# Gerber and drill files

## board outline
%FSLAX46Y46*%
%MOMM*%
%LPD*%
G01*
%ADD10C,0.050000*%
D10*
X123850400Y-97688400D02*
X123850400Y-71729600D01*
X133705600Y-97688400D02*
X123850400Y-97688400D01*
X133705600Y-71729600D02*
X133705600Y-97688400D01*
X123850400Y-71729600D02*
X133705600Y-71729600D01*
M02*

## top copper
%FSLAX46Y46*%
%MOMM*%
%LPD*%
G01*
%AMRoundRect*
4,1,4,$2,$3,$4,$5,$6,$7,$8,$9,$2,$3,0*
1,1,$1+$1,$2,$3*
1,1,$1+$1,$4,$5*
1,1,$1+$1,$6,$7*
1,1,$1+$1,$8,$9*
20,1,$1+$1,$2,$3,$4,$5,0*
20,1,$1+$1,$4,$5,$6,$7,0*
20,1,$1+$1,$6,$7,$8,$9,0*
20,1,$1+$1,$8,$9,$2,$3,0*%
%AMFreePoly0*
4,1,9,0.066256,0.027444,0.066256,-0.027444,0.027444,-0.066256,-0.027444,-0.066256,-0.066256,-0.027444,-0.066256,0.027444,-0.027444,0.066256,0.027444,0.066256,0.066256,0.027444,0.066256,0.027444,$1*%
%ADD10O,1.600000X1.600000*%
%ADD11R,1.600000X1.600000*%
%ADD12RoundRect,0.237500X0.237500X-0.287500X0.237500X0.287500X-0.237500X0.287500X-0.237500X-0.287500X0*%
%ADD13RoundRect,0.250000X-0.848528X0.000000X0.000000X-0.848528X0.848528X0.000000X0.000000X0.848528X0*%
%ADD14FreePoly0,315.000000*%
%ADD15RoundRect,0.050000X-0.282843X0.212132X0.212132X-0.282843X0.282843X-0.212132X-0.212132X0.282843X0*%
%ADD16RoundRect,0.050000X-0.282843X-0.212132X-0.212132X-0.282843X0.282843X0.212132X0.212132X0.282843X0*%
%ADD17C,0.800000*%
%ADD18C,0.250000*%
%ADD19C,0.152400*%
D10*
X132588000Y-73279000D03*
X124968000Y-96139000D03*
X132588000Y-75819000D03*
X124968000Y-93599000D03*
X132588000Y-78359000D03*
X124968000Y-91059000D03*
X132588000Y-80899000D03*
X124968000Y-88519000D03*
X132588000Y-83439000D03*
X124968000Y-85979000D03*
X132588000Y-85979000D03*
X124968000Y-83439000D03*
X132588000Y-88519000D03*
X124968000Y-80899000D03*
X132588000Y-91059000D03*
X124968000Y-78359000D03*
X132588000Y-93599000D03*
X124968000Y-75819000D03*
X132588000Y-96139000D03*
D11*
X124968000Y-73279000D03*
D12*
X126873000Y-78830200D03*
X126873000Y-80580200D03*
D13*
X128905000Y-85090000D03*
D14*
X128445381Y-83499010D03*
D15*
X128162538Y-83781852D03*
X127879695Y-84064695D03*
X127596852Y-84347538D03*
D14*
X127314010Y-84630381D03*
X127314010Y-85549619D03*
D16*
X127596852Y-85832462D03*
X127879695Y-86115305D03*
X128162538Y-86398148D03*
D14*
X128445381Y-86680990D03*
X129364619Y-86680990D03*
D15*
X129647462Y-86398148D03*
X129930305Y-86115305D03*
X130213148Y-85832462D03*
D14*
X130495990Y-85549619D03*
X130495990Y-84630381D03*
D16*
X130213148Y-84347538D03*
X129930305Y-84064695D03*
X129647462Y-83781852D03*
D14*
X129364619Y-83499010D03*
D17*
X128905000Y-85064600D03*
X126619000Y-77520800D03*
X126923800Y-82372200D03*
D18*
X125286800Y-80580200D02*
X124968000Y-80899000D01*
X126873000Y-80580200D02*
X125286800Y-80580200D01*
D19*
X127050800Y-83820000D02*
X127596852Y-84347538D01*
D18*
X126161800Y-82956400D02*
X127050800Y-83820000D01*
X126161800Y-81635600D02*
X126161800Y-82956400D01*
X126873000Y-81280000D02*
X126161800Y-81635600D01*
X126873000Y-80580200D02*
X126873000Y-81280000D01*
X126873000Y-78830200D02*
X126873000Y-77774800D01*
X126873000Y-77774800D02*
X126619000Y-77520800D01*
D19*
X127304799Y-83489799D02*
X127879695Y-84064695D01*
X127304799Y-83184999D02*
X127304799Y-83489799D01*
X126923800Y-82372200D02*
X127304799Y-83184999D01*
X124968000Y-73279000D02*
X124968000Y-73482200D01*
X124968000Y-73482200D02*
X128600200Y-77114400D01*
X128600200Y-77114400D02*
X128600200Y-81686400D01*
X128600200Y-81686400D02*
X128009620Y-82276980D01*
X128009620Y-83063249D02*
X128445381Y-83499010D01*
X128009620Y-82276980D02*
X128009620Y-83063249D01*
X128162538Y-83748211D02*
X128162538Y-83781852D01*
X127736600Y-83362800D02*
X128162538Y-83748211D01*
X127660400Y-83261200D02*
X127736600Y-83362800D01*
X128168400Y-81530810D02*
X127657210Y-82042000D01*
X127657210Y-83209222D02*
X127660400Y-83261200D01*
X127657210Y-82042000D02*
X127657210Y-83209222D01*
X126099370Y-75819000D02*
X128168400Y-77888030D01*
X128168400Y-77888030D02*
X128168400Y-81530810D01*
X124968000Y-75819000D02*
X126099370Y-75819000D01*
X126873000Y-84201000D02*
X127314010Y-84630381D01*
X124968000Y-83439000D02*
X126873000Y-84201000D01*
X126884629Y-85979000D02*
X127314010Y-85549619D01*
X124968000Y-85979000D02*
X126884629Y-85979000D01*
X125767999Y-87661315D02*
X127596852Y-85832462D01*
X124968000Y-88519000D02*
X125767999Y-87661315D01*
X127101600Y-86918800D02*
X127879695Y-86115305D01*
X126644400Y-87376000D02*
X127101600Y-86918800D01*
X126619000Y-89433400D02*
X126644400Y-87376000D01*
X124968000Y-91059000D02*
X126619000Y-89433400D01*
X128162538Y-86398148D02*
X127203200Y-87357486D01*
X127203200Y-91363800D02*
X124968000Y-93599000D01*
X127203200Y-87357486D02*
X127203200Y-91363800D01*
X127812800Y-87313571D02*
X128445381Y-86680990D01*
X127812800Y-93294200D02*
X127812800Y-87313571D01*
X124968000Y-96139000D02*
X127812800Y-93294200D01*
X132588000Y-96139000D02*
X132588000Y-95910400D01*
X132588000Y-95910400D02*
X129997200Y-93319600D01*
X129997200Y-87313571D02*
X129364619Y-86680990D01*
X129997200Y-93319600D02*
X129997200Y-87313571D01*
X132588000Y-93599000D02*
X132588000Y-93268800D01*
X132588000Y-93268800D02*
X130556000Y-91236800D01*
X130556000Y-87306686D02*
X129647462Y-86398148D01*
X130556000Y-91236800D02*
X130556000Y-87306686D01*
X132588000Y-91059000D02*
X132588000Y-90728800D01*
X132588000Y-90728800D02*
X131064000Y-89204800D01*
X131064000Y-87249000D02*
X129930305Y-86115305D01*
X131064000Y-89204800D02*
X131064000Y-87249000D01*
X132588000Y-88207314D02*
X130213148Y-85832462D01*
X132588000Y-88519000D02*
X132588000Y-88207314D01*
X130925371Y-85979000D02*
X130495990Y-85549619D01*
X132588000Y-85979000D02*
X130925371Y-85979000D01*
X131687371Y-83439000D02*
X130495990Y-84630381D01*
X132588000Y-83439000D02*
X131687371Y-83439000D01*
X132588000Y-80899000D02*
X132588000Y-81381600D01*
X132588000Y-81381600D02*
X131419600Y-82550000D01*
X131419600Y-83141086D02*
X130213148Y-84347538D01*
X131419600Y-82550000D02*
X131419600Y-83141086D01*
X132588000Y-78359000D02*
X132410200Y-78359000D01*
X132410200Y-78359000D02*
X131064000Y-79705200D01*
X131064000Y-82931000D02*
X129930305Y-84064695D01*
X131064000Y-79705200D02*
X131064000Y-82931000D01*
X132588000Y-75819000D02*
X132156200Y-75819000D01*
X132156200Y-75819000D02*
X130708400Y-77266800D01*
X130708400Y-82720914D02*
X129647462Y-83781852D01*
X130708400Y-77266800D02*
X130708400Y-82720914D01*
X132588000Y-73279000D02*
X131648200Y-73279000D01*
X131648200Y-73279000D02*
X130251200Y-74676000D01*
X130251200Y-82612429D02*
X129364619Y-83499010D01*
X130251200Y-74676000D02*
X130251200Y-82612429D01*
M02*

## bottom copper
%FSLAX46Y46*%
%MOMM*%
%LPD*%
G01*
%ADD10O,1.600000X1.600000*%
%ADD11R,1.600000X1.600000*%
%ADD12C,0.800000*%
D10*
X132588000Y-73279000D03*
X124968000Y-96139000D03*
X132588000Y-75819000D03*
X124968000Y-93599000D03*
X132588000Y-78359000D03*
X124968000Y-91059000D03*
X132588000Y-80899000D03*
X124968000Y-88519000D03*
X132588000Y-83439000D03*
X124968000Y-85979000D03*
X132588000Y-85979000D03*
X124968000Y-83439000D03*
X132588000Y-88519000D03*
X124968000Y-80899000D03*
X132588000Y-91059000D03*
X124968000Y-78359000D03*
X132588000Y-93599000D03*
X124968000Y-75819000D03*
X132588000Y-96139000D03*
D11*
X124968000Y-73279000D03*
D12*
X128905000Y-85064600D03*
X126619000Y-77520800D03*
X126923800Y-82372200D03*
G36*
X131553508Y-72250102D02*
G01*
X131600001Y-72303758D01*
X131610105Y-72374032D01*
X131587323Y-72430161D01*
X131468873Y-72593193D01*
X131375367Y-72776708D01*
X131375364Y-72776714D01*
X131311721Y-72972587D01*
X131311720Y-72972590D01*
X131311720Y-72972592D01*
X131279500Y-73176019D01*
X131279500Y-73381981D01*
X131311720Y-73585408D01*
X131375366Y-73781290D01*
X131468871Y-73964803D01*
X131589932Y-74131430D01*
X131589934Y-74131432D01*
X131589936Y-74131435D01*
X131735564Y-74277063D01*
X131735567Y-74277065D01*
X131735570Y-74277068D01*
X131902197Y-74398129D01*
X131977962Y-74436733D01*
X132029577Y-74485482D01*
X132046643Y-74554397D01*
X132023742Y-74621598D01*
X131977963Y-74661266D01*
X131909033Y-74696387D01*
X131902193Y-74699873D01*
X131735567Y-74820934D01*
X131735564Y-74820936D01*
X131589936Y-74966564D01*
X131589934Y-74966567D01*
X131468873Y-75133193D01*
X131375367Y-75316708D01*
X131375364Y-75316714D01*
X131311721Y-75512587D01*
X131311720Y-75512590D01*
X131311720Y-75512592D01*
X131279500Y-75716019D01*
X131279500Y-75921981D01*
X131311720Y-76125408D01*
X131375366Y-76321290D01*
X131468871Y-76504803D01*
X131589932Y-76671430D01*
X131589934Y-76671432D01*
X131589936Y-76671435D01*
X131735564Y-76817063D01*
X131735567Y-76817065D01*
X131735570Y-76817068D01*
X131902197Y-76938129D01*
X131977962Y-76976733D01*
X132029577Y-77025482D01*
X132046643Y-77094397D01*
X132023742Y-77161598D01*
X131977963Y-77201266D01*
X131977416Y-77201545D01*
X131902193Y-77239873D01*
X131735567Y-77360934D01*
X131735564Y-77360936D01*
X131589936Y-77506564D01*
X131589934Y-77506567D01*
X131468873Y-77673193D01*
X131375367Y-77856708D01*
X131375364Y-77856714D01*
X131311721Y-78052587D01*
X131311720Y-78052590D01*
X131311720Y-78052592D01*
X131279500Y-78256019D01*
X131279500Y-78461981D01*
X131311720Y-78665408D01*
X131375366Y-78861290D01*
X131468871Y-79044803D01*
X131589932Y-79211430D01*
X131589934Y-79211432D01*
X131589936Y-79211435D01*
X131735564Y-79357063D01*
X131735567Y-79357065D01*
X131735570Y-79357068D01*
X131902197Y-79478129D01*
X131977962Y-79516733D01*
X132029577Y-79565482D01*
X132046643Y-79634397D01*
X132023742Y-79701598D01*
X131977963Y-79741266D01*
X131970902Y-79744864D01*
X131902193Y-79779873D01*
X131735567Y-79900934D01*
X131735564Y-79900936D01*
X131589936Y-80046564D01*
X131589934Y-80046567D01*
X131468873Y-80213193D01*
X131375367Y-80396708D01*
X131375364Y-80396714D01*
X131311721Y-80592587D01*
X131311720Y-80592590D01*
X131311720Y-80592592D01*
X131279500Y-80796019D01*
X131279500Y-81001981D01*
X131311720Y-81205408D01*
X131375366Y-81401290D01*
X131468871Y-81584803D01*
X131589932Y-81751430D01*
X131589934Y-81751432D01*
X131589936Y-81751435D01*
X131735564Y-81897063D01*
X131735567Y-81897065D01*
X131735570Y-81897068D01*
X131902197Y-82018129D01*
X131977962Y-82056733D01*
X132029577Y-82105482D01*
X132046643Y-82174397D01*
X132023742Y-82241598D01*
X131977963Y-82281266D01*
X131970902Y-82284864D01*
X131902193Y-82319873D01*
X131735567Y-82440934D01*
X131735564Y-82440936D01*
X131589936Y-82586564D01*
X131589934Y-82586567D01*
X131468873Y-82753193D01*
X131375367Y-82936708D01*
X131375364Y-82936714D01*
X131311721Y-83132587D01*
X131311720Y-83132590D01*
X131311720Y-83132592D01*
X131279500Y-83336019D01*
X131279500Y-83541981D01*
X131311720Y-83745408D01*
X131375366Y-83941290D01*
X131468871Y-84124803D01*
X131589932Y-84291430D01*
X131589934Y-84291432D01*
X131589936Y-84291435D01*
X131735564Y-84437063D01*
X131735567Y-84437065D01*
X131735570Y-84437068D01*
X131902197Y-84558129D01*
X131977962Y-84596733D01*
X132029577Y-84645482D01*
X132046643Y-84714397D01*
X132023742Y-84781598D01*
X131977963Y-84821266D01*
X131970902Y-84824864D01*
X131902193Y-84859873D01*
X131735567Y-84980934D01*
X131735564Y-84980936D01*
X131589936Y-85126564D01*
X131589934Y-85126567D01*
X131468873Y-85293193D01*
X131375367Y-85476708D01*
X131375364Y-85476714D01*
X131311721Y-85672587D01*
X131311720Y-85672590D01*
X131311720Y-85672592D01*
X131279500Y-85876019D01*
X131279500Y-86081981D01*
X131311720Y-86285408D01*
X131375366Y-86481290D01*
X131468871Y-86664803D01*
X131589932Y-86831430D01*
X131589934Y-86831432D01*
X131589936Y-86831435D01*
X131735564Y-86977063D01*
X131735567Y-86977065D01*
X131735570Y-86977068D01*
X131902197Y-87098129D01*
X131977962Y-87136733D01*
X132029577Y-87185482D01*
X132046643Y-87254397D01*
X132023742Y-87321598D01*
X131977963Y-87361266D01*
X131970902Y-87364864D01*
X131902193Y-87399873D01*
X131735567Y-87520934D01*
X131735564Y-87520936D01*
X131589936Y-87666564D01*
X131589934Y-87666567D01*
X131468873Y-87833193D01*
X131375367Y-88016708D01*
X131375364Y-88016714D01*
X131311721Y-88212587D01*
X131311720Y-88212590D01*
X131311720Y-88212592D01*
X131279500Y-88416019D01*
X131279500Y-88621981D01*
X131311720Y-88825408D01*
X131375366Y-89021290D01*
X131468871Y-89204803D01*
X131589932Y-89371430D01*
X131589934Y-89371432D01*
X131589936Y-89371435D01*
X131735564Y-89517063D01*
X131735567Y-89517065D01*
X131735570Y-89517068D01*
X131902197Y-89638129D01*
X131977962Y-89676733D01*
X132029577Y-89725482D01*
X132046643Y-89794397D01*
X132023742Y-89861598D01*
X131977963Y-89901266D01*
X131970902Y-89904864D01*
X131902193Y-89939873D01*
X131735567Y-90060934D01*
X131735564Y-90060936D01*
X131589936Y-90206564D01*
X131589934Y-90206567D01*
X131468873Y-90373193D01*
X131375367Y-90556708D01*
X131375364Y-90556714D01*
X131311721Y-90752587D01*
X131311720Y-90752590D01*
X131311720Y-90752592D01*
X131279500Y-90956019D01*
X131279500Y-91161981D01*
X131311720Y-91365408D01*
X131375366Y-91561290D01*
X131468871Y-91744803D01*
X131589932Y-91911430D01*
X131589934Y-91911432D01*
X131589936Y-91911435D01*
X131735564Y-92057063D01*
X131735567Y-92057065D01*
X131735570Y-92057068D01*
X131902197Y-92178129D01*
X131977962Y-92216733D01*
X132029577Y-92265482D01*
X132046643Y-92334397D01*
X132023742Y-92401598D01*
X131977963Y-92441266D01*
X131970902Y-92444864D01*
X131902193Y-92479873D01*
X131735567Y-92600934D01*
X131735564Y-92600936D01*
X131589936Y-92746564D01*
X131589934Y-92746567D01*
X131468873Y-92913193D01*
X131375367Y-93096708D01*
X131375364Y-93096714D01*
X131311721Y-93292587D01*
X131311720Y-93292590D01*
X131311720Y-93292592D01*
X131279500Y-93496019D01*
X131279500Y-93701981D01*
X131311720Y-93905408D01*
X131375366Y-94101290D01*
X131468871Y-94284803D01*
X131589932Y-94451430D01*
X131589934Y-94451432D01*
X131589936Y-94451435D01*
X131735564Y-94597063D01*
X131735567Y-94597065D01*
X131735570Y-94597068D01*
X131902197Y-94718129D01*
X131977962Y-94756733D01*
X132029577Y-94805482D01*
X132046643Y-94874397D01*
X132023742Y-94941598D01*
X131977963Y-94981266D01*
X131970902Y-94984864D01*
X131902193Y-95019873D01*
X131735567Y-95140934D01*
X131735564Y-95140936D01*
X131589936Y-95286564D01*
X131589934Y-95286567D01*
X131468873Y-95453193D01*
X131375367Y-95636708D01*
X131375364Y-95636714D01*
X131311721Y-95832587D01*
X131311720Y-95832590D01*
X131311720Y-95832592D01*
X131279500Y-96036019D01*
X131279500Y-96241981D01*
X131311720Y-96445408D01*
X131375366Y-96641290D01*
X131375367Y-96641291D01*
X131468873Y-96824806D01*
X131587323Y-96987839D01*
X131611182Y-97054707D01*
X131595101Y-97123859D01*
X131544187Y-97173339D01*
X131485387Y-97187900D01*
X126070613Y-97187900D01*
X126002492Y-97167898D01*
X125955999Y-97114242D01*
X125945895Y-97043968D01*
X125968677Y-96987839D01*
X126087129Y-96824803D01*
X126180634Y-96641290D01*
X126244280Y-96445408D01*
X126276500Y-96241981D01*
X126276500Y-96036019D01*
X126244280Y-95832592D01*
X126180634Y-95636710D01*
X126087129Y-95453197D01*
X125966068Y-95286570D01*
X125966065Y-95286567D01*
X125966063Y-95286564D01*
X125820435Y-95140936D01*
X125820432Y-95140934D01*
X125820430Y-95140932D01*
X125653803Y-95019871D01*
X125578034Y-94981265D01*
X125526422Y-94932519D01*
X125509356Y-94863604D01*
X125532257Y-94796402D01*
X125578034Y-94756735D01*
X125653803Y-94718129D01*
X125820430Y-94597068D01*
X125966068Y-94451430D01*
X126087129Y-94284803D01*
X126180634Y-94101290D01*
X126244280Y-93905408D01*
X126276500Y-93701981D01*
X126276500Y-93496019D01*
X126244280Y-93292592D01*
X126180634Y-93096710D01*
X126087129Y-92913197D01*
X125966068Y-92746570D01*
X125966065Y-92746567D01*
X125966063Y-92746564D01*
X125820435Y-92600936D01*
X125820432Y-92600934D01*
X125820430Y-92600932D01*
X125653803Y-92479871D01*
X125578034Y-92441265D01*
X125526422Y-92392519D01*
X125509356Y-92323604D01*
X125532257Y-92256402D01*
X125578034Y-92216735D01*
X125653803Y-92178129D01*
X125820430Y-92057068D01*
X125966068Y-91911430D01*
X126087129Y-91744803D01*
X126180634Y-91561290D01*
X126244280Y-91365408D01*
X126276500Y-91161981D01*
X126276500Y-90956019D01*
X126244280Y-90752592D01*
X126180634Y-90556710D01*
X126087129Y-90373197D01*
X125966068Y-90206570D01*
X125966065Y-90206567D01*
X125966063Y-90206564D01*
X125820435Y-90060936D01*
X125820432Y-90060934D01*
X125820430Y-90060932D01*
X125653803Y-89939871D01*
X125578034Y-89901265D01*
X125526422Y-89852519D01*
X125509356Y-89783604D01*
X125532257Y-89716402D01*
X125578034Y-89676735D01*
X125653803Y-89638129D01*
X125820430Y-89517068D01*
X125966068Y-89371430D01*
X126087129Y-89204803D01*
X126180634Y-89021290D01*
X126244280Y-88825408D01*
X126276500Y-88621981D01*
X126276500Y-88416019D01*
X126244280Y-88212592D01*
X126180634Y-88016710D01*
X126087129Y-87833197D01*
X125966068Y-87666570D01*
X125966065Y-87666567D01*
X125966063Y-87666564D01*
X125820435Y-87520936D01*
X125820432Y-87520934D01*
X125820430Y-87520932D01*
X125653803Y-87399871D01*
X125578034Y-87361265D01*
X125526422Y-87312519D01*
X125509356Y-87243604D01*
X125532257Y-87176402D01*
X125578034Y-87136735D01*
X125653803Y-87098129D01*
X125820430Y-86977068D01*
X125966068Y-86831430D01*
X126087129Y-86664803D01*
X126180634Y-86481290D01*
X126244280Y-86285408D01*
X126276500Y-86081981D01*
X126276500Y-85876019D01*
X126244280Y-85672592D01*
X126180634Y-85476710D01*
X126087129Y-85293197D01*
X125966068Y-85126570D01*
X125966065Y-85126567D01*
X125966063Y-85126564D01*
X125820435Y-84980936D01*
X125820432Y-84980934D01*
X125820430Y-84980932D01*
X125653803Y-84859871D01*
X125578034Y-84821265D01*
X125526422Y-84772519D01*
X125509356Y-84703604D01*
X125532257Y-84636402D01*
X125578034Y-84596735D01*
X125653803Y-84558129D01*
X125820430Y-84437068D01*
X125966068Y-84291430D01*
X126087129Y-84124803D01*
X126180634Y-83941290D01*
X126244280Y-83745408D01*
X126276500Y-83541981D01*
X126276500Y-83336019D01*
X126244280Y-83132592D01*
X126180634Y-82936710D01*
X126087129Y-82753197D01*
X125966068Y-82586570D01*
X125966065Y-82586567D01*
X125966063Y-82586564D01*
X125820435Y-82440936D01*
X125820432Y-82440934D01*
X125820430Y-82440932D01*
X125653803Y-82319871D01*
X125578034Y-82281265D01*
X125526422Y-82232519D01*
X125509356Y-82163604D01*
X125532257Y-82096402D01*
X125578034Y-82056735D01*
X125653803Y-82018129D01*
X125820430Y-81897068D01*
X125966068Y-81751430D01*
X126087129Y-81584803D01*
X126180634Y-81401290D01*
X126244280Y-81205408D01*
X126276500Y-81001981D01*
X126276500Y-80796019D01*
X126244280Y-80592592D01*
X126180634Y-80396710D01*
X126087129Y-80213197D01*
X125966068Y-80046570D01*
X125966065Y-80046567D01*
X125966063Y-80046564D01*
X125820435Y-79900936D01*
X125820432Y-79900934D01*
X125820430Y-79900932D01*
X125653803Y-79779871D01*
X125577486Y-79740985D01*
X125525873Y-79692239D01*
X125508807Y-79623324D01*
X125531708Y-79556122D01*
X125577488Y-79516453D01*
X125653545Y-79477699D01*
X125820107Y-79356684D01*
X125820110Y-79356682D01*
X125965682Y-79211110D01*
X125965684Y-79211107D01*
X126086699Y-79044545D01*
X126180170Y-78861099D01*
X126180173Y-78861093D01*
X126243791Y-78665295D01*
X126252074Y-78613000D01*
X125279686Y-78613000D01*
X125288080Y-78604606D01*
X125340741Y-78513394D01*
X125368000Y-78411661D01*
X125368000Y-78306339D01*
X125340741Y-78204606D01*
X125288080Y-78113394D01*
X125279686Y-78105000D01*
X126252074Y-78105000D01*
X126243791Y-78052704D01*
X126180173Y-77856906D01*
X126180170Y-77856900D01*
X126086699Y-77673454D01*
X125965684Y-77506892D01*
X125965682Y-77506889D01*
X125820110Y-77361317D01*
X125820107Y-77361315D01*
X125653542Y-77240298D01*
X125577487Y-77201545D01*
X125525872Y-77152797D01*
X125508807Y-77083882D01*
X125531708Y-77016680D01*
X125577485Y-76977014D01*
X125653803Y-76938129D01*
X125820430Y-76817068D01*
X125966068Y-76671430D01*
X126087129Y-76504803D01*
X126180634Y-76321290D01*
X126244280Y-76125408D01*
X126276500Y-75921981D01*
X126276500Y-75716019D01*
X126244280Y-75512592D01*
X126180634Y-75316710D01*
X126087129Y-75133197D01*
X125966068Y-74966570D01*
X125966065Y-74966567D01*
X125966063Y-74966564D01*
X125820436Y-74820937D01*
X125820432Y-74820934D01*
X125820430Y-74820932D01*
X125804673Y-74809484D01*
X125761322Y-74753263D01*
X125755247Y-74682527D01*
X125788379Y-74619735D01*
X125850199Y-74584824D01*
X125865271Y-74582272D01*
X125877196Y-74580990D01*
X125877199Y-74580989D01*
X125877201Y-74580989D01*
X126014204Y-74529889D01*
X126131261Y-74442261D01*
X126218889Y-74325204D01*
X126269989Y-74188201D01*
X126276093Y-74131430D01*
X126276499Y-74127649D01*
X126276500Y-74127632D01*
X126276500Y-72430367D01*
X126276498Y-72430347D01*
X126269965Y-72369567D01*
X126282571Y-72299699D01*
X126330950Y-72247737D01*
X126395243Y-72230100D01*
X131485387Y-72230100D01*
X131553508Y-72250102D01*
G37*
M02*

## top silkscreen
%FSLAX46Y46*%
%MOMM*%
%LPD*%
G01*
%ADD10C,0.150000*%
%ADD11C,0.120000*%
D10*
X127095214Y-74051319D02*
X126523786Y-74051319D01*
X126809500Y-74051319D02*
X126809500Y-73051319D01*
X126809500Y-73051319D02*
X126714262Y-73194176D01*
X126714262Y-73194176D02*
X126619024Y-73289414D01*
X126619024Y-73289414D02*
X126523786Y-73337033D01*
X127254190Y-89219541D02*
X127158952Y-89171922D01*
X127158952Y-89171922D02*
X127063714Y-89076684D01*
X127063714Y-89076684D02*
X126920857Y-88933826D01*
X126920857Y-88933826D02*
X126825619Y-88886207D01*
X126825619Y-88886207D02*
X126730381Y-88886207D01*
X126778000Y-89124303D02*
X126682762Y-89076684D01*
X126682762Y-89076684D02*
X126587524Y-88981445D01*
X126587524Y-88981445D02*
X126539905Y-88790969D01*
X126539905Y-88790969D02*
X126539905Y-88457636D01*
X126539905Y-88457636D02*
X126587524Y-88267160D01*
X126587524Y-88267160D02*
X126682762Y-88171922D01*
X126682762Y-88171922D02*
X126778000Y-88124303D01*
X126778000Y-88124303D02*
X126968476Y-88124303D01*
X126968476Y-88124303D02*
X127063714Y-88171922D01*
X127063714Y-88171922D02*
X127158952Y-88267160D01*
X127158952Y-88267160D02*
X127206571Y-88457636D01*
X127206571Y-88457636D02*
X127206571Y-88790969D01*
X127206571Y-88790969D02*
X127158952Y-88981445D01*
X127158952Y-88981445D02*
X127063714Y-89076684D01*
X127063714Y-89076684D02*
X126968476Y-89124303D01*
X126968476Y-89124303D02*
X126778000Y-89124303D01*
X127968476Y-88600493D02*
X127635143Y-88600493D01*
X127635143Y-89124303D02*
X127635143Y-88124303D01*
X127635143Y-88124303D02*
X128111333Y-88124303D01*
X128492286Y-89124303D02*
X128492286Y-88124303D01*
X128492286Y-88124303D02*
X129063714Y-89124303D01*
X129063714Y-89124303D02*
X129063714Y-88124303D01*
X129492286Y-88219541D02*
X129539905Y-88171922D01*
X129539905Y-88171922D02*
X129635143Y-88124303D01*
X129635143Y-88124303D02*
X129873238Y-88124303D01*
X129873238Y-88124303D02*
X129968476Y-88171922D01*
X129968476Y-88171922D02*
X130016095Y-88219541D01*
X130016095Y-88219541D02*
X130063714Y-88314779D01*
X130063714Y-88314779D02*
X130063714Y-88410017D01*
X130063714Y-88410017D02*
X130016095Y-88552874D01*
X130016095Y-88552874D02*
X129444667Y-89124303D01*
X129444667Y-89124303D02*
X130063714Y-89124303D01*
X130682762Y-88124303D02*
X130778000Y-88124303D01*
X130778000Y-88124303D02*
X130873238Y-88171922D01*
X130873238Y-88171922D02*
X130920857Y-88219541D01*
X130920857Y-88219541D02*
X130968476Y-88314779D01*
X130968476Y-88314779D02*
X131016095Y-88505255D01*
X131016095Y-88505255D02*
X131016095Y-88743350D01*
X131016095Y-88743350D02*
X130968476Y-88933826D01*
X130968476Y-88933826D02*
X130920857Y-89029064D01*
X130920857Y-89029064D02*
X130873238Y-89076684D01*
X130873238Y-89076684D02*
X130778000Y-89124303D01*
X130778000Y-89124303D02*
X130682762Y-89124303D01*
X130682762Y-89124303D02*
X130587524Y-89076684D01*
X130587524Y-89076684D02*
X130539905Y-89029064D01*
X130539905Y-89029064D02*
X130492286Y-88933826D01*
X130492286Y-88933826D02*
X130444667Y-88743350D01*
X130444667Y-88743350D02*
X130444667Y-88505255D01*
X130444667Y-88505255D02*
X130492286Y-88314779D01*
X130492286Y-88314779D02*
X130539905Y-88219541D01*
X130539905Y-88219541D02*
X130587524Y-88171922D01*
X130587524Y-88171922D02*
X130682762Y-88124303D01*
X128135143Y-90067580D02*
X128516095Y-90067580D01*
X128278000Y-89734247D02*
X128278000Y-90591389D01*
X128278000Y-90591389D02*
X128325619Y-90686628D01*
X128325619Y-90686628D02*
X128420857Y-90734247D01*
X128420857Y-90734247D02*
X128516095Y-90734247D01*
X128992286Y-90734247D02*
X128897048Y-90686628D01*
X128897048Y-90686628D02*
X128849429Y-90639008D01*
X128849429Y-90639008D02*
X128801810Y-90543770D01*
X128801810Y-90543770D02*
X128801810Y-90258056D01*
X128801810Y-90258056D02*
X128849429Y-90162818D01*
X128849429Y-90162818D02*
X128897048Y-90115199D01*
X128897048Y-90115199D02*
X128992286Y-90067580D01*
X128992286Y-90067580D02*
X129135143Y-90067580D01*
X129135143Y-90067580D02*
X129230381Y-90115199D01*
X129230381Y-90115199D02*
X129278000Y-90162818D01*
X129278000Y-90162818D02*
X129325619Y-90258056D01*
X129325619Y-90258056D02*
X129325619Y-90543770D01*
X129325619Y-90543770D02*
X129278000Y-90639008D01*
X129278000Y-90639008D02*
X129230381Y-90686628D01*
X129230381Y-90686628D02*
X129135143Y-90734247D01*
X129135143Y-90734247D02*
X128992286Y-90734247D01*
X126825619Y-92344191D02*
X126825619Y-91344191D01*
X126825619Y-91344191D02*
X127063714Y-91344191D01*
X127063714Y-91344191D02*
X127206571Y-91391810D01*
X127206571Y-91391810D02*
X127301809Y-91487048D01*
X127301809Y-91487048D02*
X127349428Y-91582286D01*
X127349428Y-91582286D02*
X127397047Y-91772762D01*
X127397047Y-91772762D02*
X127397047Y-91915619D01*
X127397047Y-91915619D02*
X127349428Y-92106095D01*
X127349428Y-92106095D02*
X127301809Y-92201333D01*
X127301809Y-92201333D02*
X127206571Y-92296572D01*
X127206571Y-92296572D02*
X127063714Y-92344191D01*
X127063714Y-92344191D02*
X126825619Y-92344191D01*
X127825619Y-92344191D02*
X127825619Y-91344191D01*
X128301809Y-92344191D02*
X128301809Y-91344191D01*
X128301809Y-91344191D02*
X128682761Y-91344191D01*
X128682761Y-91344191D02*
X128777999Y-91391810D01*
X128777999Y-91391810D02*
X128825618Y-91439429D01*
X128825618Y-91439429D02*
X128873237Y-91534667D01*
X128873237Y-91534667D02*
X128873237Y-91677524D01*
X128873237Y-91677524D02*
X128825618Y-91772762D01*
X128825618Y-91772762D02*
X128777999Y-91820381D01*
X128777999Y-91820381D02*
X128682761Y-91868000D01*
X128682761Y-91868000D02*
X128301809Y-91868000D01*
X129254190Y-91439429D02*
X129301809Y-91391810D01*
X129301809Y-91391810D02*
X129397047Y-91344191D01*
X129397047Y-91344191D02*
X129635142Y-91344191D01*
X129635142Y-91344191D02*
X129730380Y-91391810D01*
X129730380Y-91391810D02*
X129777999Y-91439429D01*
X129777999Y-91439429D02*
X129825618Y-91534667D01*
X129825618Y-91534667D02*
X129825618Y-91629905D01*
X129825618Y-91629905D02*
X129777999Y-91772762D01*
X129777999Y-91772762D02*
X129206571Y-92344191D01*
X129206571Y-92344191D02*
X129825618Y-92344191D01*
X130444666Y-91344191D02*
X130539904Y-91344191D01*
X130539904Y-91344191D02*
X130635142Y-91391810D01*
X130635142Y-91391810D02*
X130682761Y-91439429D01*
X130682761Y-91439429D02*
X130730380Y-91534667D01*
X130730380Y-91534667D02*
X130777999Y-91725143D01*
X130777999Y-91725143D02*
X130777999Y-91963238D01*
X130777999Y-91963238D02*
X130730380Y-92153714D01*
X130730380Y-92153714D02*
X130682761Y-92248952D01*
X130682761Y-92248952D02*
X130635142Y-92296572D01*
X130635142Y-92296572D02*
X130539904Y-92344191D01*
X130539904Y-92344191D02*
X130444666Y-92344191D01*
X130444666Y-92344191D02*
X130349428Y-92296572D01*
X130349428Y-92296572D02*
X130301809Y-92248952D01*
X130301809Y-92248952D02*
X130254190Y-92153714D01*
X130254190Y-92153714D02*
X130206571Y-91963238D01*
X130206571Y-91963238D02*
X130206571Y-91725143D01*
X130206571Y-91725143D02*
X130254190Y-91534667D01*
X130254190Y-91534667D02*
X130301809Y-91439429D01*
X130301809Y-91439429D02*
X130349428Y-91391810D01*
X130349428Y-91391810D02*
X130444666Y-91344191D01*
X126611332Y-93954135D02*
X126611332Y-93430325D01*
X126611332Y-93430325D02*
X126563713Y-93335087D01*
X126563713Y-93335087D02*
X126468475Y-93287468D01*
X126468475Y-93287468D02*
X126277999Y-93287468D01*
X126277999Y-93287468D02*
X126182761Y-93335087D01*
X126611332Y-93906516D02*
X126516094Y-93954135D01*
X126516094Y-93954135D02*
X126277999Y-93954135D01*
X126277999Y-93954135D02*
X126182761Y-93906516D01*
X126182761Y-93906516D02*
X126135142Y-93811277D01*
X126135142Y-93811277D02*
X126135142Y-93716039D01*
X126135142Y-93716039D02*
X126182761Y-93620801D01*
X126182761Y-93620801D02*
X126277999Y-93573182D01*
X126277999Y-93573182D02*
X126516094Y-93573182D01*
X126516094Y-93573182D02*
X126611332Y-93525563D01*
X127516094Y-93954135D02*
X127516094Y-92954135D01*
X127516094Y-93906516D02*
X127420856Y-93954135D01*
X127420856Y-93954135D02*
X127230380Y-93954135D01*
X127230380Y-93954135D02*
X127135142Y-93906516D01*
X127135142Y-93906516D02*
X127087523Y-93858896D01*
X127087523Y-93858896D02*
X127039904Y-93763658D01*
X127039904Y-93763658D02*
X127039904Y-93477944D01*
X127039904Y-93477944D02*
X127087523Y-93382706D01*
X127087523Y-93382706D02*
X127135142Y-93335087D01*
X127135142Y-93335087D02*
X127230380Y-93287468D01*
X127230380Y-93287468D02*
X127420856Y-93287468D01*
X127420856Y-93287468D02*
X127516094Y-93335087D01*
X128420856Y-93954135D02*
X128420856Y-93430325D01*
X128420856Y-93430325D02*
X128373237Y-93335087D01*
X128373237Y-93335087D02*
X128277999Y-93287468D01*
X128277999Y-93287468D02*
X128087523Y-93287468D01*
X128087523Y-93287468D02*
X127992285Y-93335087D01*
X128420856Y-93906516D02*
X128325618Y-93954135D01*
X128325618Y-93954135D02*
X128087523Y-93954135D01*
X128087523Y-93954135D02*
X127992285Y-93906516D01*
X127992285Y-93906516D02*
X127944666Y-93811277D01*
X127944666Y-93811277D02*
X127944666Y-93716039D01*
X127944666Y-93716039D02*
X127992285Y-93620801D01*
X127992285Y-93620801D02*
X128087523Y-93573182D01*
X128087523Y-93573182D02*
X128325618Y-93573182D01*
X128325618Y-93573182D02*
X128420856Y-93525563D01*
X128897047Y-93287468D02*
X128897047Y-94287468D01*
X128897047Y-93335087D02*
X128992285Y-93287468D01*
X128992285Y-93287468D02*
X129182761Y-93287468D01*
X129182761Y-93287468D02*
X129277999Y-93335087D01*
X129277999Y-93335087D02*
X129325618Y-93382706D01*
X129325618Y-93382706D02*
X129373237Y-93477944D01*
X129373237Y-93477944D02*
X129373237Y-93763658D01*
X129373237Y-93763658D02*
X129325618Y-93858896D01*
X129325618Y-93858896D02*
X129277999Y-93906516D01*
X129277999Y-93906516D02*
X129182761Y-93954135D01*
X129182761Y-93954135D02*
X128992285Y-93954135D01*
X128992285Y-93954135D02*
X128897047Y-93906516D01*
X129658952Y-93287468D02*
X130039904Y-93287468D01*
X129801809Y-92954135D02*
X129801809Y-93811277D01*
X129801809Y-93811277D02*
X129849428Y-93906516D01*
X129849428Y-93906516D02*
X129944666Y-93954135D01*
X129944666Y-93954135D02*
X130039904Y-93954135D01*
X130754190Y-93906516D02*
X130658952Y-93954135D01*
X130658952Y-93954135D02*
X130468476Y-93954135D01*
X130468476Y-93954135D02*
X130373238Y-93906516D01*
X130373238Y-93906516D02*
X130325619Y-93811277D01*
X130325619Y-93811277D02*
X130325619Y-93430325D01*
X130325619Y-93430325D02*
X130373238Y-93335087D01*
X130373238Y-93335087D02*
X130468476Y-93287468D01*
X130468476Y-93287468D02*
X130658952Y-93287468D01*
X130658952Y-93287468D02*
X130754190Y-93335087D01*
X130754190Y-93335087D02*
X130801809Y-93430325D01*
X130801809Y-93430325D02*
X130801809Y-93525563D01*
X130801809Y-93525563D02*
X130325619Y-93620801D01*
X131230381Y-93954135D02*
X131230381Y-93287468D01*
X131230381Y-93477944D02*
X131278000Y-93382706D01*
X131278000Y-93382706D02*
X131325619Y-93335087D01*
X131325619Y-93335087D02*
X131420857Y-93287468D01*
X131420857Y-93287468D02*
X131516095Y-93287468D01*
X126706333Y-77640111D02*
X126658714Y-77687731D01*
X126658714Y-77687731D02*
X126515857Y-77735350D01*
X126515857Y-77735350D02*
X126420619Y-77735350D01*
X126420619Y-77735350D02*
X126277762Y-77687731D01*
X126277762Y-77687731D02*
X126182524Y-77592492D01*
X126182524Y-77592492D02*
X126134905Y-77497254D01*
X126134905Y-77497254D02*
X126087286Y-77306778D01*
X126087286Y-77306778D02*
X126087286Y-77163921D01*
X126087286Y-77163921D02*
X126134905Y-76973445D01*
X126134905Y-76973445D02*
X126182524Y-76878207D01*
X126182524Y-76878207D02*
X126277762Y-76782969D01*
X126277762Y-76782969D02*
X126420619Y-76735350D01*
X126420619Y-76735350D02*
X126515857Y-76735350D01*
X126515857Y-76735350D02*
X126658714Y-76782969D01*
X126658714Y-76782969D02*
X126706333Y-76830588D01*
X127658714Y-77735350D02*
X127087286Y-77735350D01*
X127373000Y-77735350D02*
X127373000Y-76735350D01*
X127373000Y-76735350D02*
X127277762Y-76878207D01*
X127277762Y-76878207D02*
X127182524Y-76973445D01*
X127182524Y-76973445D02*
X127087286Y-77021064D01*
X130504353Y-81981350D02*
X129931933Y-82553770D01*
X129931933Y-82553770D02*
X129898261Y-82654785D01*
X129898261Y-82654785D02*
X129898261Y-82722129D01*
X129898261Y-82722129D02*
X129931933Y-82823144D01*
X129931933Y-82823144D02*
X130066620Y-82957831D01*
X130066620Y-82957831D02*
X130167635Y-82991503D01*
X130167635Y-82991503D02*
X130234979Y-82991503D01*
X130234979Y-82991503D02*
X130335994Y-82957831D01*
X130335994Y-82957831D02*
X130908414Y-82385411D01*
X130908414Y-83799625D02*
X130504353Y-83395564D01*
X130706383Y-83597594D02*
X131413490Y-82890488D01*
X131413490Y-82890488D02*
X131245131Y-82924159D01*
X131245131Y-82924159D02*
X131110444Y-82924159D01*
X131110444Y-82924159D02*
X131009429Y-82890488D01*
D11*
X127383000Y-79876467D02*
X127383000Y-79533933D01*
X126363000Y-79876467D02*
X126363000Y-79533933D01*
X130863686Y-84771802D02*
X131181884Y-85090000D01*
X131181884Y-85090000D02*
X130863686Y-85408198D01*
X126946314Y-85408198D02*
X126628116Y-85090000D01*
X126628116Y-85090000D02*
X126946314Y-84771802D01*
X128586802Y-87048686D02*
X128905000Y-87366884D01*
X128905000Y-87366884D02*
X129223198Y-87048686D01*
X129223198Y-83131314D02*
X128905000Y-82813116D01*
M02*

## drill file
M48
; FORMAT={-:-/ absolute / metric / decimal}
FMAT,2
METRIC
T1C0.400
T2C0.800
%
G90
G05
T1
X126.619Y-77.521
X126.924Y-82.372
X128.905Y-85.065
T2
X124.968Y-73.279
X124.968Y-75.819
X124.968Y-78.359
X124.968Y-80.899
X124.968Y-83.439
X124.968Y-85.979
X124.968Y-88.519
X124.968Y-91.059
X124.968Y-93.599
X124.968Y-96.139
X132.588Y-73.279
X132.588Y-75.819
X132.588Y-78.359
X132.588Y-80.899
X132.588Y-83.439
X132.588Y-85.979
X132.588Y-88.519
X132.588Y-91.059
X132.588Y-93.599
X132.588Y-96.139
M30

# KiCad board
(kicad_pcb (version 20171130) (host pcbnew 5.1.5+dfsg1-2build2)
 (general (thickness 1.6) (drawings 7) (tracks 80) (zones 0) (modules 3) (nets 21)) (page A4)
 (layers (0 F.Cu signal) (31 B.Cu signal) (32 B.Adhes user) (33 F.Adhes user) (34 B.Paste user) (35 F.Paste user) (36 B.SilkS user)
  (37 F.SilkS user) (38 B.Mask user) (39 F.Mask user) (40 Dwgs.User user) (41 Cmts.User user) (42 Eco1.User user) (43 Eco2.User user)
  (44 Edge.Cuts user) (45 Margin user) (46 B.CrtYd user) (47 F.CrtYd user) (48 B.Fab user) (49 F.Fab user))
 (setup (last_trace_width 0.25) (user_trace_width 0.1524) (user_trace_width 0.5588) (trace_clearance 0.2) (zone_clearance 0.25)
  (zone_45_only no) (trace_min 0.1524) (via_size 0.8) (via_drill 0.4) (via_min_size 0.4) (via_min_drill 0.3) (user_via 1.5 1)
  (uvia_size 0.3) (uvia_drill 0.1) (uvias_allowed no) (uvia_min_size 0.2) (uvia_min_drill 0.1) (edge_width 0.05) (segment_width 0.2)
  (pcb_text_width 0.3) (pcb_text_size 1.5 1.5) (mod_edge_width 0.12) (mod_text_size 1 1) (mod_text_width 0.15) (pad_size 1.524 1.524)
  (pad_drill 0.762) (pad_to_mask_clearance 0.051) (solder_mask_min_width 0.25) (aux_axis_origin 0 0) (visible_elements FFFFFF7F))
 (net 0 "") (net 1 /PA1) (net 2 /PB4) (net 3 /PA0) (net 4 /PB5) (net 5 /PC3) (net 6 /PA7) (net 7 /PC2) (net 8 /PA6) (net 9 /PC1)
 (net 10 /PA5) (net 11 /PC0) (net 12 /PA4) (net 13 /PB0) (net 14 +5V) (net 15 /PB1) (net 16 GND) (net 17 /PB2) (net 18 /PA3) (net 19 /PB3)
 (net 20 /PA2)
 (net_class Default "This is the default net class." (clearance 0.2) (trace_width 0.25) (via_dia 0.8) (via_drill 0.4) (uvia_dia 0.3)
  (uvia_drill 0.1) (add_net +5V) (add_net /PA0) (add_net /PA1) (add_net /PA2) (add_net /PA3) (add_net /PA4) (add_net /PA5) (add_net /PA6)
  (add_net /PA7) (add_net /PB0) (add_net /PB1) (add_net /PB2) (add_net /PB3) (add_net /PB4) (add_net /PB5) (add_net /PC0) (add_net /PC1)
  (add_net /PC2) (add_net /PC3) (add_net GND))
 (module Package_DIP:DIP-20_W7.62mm (layer F.Cu) (at 124.968 73.279)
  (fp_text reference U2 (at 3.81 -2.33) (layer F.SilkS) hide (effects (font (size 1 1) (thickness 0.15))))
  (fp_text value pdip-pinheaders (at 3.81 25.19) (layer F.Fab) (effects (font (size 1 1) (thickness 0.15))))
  (pad 20 thru_hole oval (at 7.62 0) (size 1.6 1.6) (drill 0.8) (layers *.Cu *.Mask) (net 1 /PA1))
  (pad 10 thru_hole oval (at 0 22.86) (size 1.6 1.6) (drill 0.8) (layers *.Cu *.Mask) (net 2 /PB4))
  (pad 19 thru_hole oval (at 7.62 2.54) (size 1.6 1.6) (drill 0.8) (layers *.Cu *.Mask) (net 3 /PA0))
  (pad 9 thru_hole oval (at 0 20.32) (size 1.6 1.6) (drill 0.8) (layers *.Cu *.Mask) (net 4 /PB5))
  (pad 18 thru_hole oval (at 7.62 5.08) (size 1.6 1.6) (drill 0.8) (layers *.Cu *.Mask) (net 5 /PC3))
  (pad 8 thru_hole oval (at 0 17.78) (size 1.6 1.6) (drill 0.8) (layers *.Cu *.Mask) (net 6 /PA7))
  (pad 17 thru_hole oval (at 7.62 7.62) (size 1.6 1.6) (drill 0.8) (layers *.Cu *.Mask) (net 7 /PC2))
  (pad 7 thru_hole oval (at 0 15.24) (size 1.6 1.6) (drill 0.8) (layers *.Cu *.Mask) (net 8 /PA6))
  (pad 16 thru_hole oval (at 7.62 10.16) (size 1.6 1.6) (drill 0.8) (layers *.Cu *.Mask) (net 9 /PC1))
  (pad 6 thru_hole oval (at 0 12.7) (size 1.6 1.6) (drill 0.8) (layers *.Cu *.Mask) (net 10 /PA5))
  (pad 15 thru_hole oval (at 7.62 12.7) (size 1.6 1.6) (drill 0.8) (layers *.Cu *.Mask) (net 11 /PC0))
  (pad 5 thru_hole oval (at 0 10.16) (size 1.6 1.6) (drill 0.8) (layers *.Cu *.Mask) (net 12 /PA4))
  (pad 14 thru_hole oval (at 7.62 15.24) (size 1.6 1.6) (drill 0.8) (layers *.Cu *.Mask) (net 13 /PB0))
  (pad 4 thru_hole oval (at 0 7.62) (size 1.6 1.6) (drill 0.8) (layers *.Cu *.Mask) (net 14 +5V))
  (pad 13 thru_hole oval (at 7.62 17.78) (size 1.6 1.6) (drill 0.8) (layers *.Cu *.Mask) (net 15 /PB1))
  (pad 3 thru_hole oval (at 0 5.08) (size 1.6 1.6) (drill 0.8) (layers *.Cu *.Mask) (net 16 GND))
  (pad 12 thru_hole oval (at 7.62 20.32) (size 1.6 1.6) (drill 0.8) (layers *.Cu *.Mask) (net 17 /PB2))
  (pad 2 thru_hole oval (at 0 2.54) (size 1.6 1.6) (drill 0.8) (layers *.Cu *.Mask) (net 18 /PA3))
  (pad 11 thru_hole oval (at 7.62 22.86) (size 1.6 1.6) (drill 0.8) (layers *.Cu *.Mask) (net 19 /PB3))
  (pad 1 thru_hole rect (at 0 0) (size 1.6 1.6) (drill 0.8) (layers *.Cu *.Mask) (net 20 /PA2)))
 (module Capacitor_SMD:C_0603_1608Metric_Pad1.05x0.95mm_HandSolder (layer F.Cu) (at 126.873 79.7052 90)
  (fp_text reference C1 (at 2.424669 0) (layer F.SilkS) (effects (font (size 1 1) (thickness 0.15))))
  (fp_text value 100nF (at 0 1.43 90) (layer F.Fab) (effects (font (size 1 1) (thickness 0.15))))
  (fp_line (start -0.171267 0.51) (end 0.171267 0.51) (layer F.SilkS) (width 0.12))
  (fp_line (start -0.171267 -0.51) (end 0.171267 -0.51) (layer F.SilkS) (width 0.12))
  (pad 2 smd roundrect (at 0.875 0 90) (size 1.05 0.95) (layers F.Cu F.Paste F.Mask) (roundrect_rratio 0.25) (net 16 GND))
  (pad 1 smd roundrect (at -0.875 0 90) (size 1.05 0.95) (layers F.Cu F.Paste F.Mask) (roundrect_rratio 0.25) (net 14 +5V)))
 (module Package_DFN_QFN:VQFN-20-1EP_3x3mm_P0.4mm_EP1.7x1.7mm (layer F.Cu) (at 128.905 85.09 315)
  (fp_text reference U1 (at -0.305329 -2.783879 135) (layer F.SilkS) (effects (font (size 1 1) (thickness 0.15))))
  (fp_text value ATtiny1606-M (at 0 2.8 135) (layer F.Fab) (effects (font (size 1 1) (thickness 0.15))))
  (fp_line (start 1.16 -1.61) (end 1.61 -1.61) (layer F.SilkS) (width 0.12))
  (fp_line (start 1.61 -1.61) (end 1.61 -1.16) (layer F.SilkS) (width 0.12))
  (fp_line (start -1.16 1.61) (end -1.61 1.61) (layer F.SilkS) (width 0.12))
  (fp_line (start -1.61 1.61) (end -1.61 1.16) (layer F.SilkS) (width 0.12))
  (fp_line (start 1.16 1.61) (end 1.61 1.61) (layer F.SilkS) (width 0.12))
  (fp_line (start 1.61 1.61) (end 1.61 1.16) (layer F.SilkS) (width 0.12))
  (fp_line (start -1.16 -1.61) (end -1.61 -1.61) (layer F.SilkS) (width 0.12))
  (pad 21 smd roundrect (at 0 0 315) (size 1.7 1.7) (layers F.Cu F.Mask) (roundrect_rratio 0.147059) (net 16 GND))
  (pad "" smd roundrect (at -0.425 -0.425 315) (size 0.69 0.69) (layers F.Paste) (roundrect_rratio 0.25))
  (pad "" smd roundrect (at -0.425 0.425 315) (size 0.69 0.69) (layers F.Paste) (roundrect_rratio 0.25))
  (pad "" smd roundrect (at 0.425 -0.425 315) (size 0.69 0.69) (layers F.Paste) (roundrect_rratio 0.25))
  (pad "" smd roundrect (at 0.425 0.425 315) (size 0.69 0.69) (layers F.Paste) (roundrect_rratio 0.25))
  (pad 1 smd custom (at -1.45 -0.8 315) (size 0.143431 0.143431) (layers F.Cu F.Paste F.Mask) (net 20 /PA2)
   (options (clearance outline) (anchor circle)) (primitives))
  (pad 2 smd roundrect (at -1.45 -0.4 315) (size 0.8 0.2) (layers F.Cu F.Paste F.Mask) (roundrect_rratio 0.25) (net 18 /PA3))
  (pad 3 smd roundrect (at -1.45 0 315) (size 0.8 0.2) (layers F.Cu F.Paste F.Mask) (roundrect_rratio 0.25) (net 16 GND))
  (pad 4 smd roundrect (at -1.45 0.4 315) (size 0.8 0.2) (layers F.Cu F.Paste F.Mask) (roundrect_rratio 0.25) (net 14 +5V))
  (pad 5 smd custom (at -1.45 0.8 315) (size 0.143431 0.143431) (layers F.Cu F.Paste F.Mask) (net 12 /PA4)
   (options (clearance outline) (anchor circle)) (primitives))
  (pad 6 smd custom (at -0.8 1.45 315) (size 0.143431 0.143431) (layers F.Cu F.Paste F.Mask) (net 10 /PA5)
   (options (clearance outline) (anchor circle)) (primitives))
  (pad 7 smd roundrect (at -0.4 1.45 315) (size 0.2 0.8) (layers F.Cu F.Paste F.Mask) (roundrect_rratio 0.25) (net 8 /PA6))
  (pad 8 smd roundrect (at 0 1.45 315) (size 0.2 0.8) (layers F.Cu F.Paste F.Mask) (roundrect_rratio 0.25) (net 6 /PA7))
  (pad 9 smd roundrect (at 0.4 1.45 315) (size 0.2 0.8) (layers F.Cu F.Paste F.Mask) (roundrect_rratio 0.25) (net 4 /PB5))
  (pad 10 smd custom (at 0.8 1.45 315) (size 0.143431 0.143431) (layers F.Cu F.Paste F.Mask) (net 2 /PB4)
   (options (clearance outline) (anchor circle)) (primitives))
  (pad 11 smd custom (at 1.45 0.8 315) (size 0.143431 0.143431) (layers F.Cu F.Paste F.Mask) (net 19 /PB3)
   (options (clearance outline) (anchor circle)) (primitives))
  (pad 12 smd roundrect (at 1.45 0.4 315) (size 0.8 0.2) (layers F.Cu F.Paste F.Mask) (roundrect_rratio 0.25) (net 17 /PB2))
  (pad 13 smd roundrect (at 1.45 0 315) (size 0.8 0.2) (layers F.Cu F.Paste F.Mask) (roundrect_rratio 0.25) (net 15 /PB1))
  (pad 14 smd roundrect (at 1.45 -0.4 315) (size 0.8 0.2) (layers F.Cu F.Paste F.Mask) (roundrect_rratio 0.25) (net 13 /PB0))
  (pad 15 smd custom (at 1.45 -0.8 315) (size 0.143431 0.143431) (layers F.Cu F.Paste F.Mask) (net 11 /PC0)
   (options (clearance outline) (anchor circle)) (primitives))
  (pad 16 smd custom (at 0.8 -1.45 315) (size 0.143431 0.143431) (layers F.Cu F.Paste F.Mask) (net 9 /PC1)
   (options (clearance outline) (anchor circle)) (primitives))
  (pad 17 smd roundrect (at 0.4 -1.45 315) (size 0.2 0.8) (layers F.Cu F.Paste F.Mask) (roundrect_rratio 0.25) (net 7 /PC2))
  (pad 18 smd roundrect (at 0 -1.45 315) (size 0.2 0.8) (layers F.Cu F.Paste F.Mask) (roundrect_rratio 0.25) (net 5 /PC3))
  (pad 19 smd roundrect (at -0.4 -1.45 315) (size 0.2 0.8) (layers F.Cu F.Paste F.Mask) (roundrect_rratio 0.25) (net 3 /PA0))
  (pad 20 smd custom (at -0.8 -1.45 315) (size 0.143431 0.143431) (layers F.Cu F.Paste F.Mask) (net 1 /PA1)
   (options (clearance outline) (anchor circle)) (primitives)))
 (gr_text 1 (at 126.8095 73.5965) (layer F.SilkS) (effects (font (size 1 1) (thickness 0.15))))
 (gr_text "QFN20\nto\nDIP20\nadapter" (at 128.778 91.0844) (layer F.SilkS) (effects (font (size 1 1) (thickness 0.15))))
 (gr_line (start 123.8504 97.6884) (end 123.8504 71.7296) (layer Edge.Cuts) (width 0.05))
 (gr_line (start 133.7056 97.6884) (end 123.8504 97.6884) (layer Edge.Cuts) (width 0.05))
 (gr_line (start 133.7056 71.7296) (end 133.7056 97.6884) (layer Edge.Cuts) (width 0.05))
 (gr_line (start 123.8504 71.7296) (end 133.7056 71.7296) (layer Edge.Cuts) (width 0.05))
 (segment (start 125.2868 80.5802) (end 124.968 80.899) (width 0.25) (layer F.Cu) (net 14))
 (segment (start 126.873 80.5802) (end 125.2868 80.5802) (width 0.25) (layer F.Cu) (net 14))
 (segment (start 127.0508 83.82) (end 127.596852 84.347538) (width 0.1524) (layer F.Cu) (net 14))
 (segment (start 126.1618 82.9564) (end 127.0508 83.82) (width 0.25) (layer F.Cu) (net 14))
 (segment (start 126.1618 81.6356) (end 126.1618 82.9564) (width 0.25) (layer F.Cu) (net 14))
 (segment (start 126.873 81.28) (end 126.1618 81.6356) (width 0.25) (layer F.Cu) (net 14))
 (segment (start 126.873 80.5802) (end 126.873 81.28) (width 0.25) (layer F.Cu) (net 14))
 (via (at 128.905 85.0646) (size 0.8) (drill 0.4) (layers F.Cu B.Cu) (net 16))
 (via (at 126.619 77.5208) (size 0.8) (drill 0.4) (layers F.Cu B.Cu) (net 16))
 (segment (start 126.873 78.8302) (end 126.873 77.7748) (width 0.25) (layer F.Cu) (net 16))
 (segment (start 126.873 77.7748) (end 126.619 77.5208) (width 0.25) (layer F.Cu) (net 16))
 (segment (start 127.304799 83.489799) (end 127.879695 84.064695) (width 0.1524) (layer F.Cu) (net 16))
 (segment (start 127.304799 83.184999) (end 127.304799 83.489799) (width 0.1524) (layer F.Cu) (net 16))
 (segment (start 126.9238 82.3722) (end 127.304799 83.184999) (width 0.1524) (layer F.Cu) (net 16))
 (via (at 126.9238 82.3722) (size 0.8) (drill 0.4) (layers F.Cu B.Cu) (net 16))
 (segment (start 124.968 73.279) (end 124.968 73.4822) (width 0.1524) (layer F.Cu) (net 20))
 (segment (start 124.968 73.4822) (end 128.6002 77.1144) (width 0.1524) (layer F.Cu) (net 20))
 (segment (start 128.6002 77.1144) (end 128.6002 81.6864) (width 0.1524) (layer F.Cu) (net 20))
 (segment (start 128.6002 81.6864) (end 128.00962 82.27698) (width 0.1524) (layer F.Cu) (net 20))
 (segment (start 128.00962 83.063249) (end 128.445381 83.49901) (width 0.1524) (layer F.Cu) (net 20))
 (segment (start 128.00962 82.27698) (end 128.00962 83.063249) (width 0.1524) (layer F.Cu) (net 20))
 (segment (start 128.162538 83.748211) (end 128.162538 83.781852) (width 0.1524) (layer F.Cu) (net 18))
 (segment (start 127.7366 83.3628) (end 128.162538 83.748211) (width 0.1524) (layer F.Cu) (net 18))
 (segment (start 127.6604 83.2612) (end 127.7366 83.3628) (width 0.1524) (layer F.Cu) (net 18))
 (segment (start 128.1684 81.53081) (end 127.65721 82.042) (width 0.1524) (layer F.Cu) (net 18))
 (segment (start 127.65721 83.209222) (end 127.6604 83.2612) (width 0.1524) (layer F.Cu) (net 18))
 (segment (start 127.65721 82.042) (end 127.65721 83.209222) (width 0.1524) (layer F.Cu) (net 18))
 (segment (start 126.09937 75.819) (end 128.1684 77.88803) (width 0.1524) (layer F.Cu) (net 18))
 (segment (start 128.1684 77.88803) (end 128.1684 81.53081) (width 0.1524) (layer F.Cu) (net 18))
 (segment (start 124.968 75.819) (end 126.09937 75.819) (width 0.1524) (layer F.Cu) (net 18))
 (segment (start 126.873 84.201) (end 127.31401 84.630381) (width 0.1524) (layer F.Cu) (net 12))
 (segment (start 124.968 83.439) (end 126.873 84.201) (width 0.1524) (layer F.Cu) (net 12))
 (segment (start 126.884629 85.979) (end 127.31401 85.549619) (width 0.1524) (layer F.Cu) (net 10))
 (segment (start 124.968 85.979) (end 126.884629 85.979) (width 0.1524) (layer F.Cu) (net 10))
 (segment (start 125.767999 87.661315) (end 127.596852 85.832462) (width 0.1524) (layer F.Cu) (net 8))
 (segment (start 124.968 88.519) (end 125.767999 87.661315) (width 0.1524) (layer F.Cu) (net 8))
 (segment (start 127.1016 86.9188) (end 127.879695 86.115305) (width 0.1524) (layer F.Cu) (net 6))
 (segment (start 126.6444 87.376) (end 127.1016 86.9188) (width 0.1524) (layer F.Cu) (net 6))
 (segment (start 126.619 89.4334) (end 126.6444 87.376) (width 0.1524) (layer F.Cu) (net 6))
 (segment (start 124.968 91.059) (end 126.619 89.4334) (width 0.1524) (layer F.Cu) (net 6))
 (segment (start 128.162538 86.398148) (end 127.2032 87.357486) (width 0.1524) (layer F.Cu) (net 4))
 (segment (start 127.2032 91.3638) (end 124.968 93.599) (width 0.1524) (layer F.Cu) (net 4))
 (segment (start 127.2032 87.357486) (end 127.2032 91.3638) (width 0.1524) (layer F.Cu) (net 4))
 (segment (start 127.8128 87.313571) (end 128.445381 86.68099) (width 0.1524) (layer F.Cu) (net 2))
 (segment (start 127.8128 93.2942) (end 127.8128 87.313571) (width 0.1524) (layer F.Cu) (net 2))
 (segment (start 124.968 96.139) (end 127.8128 93.2942) (width 0.1524) (layer F.Cu) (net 2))
 (segment (start 132.588 96.139) (end 132.588 95.9104) (width 0.1524) (layer F.Cu) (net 19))
 (segment (start 132.588 95.9104) (end 129.9972 93.3196) (width 0.1524) (layer F.Cu) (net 19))
 (segment (start 129.9972 87.313571) (end 129.364619 86.68099) (width 0.1524) (layer F.Cu) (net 19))
 (segment (start 129.9972 93.3196) (end 129.9972 87.313571) (width 0.1524) (layer F.Cu) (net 19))
 (segment (start 132.588 93.599) (end 132.588 93.2688) (width 0.1524) (layer F.Cu) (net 17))
 (segment (start 132.588 93.2688) (end 130.556 91.2368) (width 0.1524) (layer F.Cu) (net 17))
 (segment (start 130.556 87.306686) (end 129.647462 86.398148) (width 0.1524) (layer F.Cu) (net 17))
 (segment (start 130.556 91.2368) (end 130.556 87.306686) (width 0.1524) (layer F.Cu) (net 17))
 (segment (start 132.588 91.059) (end 132.588 90.7288) (width 0.1524) (layer F.Cu) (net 15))
 (segment (start 132.588 90.7288) (end 131.064 89.2048) (width 0.1524) (layer F.Cu) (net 15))
 (segment (start 131.064 87.249) (end 129.930305 86.115305) (width 0.1524) (layer F.Cu) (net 15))
 (segment (start 131.064 89.2048) (end 131.064 87.249) (width 0.1524) (layer F.Cu) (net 15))
 (segment (start 132.588 88.207314) (end 130.213148 85.832462) (width 0.1524) (layer F.Cu) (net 13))
 (segment (start 132.588 88.519) (end 132.588 88.207314) (width 0.1524) (layer F.Cu) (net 13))
 (segment (start 130.925371 85.979) (end 130.49599 85.549619) (width 0.1524) (layer F.Cu) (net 11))
 (segment (start 132.588 85.979) (end 130.925371 85.979) (width 0.1524) (layer F.Cu) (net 11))
 (segment (start 131.687371 83.439) (end 130.49599 84.630381) (width 0.1524) (layer F.Cu) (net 9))
 (segment (start 132.588 83.439) (end 131.687371 83.439) (width 0.1524) (layer F.Cu) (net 9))
 (segment (start 132.588 80.899) (end 132.588 81.3816) (width 0.1524) (layer F.Cu) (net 7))
 (segment (start 132.588 81.3816) (end 131.4196 82.55) (width 0.1524) (layer F.Cu) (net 7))
 (segment (start 131.4196 83.141086) (end 130.213148 84.347538) (width 0.1524) (layer F.Cu) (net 7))
 (segment (start 131.4196 82.55) (end 131.4196 83.141086) (width 0.1524) (layer F.Cu) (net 7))
 (segment (start 132.588 78.359) (end 132.4102 78.359) (width 0.1524) (layer F.Cu) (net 5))
 (segment (start 132.4102 78.359) (end 131.064 79.7052) (width 0.1524) (layer F.Cu) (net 5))
 (segment (start 131.064 82.931) (end 129.930305 84.064695) (width 0.1524) (layer F.Cu) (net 5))
 (segment (start 131.064 79.7052) (end 131.064 82.931) (width 0.1524) (layer F.Cu) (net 5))
 (segment (start 132.588 75.819) (end 132.1562 75.819) (width 0.1524) (layer F.Cu) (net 3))
 (segment (start 132.1562 75.819) (end 130.7084 77.2668) (width 0.1524) (layer F.Cu) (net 3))
 (segment (start 130.7084 82.720914) (end 129.647462 83.781852) (width 0.1524) (layer F.Cu) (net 3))
 (segment (start 130.7084 77.2668) (end 130.7084 82.720914) (width 0.1524) (layer F.Cu) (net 3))
 (segment (start 132.588 73.279) (end 131.6482 73.279) (width 0.1524) (layer F.Cu) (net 1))
 (segment (start 131.6482 73.279) (end 130.2512 74.676) (width 0.1524) (layer F.Cu) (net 1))
 (segment (start 130.2512 82.612429) (end 129.364619 83.49901) (width 0.1524) (layer F.Cu) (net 1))
 (segment (start 130.2512 74.676) (end 130.2512 82.612429) (width 0.1524) (layer F.Cu) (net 1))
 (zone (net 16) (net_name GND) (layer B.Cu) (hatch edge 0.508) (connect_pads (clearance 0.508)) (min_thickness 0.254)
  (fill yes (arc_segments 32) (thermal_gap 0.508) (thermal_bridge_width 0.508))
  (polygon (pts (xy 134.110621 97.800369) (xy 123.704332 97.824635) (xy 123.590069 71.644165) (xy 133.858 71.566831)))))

